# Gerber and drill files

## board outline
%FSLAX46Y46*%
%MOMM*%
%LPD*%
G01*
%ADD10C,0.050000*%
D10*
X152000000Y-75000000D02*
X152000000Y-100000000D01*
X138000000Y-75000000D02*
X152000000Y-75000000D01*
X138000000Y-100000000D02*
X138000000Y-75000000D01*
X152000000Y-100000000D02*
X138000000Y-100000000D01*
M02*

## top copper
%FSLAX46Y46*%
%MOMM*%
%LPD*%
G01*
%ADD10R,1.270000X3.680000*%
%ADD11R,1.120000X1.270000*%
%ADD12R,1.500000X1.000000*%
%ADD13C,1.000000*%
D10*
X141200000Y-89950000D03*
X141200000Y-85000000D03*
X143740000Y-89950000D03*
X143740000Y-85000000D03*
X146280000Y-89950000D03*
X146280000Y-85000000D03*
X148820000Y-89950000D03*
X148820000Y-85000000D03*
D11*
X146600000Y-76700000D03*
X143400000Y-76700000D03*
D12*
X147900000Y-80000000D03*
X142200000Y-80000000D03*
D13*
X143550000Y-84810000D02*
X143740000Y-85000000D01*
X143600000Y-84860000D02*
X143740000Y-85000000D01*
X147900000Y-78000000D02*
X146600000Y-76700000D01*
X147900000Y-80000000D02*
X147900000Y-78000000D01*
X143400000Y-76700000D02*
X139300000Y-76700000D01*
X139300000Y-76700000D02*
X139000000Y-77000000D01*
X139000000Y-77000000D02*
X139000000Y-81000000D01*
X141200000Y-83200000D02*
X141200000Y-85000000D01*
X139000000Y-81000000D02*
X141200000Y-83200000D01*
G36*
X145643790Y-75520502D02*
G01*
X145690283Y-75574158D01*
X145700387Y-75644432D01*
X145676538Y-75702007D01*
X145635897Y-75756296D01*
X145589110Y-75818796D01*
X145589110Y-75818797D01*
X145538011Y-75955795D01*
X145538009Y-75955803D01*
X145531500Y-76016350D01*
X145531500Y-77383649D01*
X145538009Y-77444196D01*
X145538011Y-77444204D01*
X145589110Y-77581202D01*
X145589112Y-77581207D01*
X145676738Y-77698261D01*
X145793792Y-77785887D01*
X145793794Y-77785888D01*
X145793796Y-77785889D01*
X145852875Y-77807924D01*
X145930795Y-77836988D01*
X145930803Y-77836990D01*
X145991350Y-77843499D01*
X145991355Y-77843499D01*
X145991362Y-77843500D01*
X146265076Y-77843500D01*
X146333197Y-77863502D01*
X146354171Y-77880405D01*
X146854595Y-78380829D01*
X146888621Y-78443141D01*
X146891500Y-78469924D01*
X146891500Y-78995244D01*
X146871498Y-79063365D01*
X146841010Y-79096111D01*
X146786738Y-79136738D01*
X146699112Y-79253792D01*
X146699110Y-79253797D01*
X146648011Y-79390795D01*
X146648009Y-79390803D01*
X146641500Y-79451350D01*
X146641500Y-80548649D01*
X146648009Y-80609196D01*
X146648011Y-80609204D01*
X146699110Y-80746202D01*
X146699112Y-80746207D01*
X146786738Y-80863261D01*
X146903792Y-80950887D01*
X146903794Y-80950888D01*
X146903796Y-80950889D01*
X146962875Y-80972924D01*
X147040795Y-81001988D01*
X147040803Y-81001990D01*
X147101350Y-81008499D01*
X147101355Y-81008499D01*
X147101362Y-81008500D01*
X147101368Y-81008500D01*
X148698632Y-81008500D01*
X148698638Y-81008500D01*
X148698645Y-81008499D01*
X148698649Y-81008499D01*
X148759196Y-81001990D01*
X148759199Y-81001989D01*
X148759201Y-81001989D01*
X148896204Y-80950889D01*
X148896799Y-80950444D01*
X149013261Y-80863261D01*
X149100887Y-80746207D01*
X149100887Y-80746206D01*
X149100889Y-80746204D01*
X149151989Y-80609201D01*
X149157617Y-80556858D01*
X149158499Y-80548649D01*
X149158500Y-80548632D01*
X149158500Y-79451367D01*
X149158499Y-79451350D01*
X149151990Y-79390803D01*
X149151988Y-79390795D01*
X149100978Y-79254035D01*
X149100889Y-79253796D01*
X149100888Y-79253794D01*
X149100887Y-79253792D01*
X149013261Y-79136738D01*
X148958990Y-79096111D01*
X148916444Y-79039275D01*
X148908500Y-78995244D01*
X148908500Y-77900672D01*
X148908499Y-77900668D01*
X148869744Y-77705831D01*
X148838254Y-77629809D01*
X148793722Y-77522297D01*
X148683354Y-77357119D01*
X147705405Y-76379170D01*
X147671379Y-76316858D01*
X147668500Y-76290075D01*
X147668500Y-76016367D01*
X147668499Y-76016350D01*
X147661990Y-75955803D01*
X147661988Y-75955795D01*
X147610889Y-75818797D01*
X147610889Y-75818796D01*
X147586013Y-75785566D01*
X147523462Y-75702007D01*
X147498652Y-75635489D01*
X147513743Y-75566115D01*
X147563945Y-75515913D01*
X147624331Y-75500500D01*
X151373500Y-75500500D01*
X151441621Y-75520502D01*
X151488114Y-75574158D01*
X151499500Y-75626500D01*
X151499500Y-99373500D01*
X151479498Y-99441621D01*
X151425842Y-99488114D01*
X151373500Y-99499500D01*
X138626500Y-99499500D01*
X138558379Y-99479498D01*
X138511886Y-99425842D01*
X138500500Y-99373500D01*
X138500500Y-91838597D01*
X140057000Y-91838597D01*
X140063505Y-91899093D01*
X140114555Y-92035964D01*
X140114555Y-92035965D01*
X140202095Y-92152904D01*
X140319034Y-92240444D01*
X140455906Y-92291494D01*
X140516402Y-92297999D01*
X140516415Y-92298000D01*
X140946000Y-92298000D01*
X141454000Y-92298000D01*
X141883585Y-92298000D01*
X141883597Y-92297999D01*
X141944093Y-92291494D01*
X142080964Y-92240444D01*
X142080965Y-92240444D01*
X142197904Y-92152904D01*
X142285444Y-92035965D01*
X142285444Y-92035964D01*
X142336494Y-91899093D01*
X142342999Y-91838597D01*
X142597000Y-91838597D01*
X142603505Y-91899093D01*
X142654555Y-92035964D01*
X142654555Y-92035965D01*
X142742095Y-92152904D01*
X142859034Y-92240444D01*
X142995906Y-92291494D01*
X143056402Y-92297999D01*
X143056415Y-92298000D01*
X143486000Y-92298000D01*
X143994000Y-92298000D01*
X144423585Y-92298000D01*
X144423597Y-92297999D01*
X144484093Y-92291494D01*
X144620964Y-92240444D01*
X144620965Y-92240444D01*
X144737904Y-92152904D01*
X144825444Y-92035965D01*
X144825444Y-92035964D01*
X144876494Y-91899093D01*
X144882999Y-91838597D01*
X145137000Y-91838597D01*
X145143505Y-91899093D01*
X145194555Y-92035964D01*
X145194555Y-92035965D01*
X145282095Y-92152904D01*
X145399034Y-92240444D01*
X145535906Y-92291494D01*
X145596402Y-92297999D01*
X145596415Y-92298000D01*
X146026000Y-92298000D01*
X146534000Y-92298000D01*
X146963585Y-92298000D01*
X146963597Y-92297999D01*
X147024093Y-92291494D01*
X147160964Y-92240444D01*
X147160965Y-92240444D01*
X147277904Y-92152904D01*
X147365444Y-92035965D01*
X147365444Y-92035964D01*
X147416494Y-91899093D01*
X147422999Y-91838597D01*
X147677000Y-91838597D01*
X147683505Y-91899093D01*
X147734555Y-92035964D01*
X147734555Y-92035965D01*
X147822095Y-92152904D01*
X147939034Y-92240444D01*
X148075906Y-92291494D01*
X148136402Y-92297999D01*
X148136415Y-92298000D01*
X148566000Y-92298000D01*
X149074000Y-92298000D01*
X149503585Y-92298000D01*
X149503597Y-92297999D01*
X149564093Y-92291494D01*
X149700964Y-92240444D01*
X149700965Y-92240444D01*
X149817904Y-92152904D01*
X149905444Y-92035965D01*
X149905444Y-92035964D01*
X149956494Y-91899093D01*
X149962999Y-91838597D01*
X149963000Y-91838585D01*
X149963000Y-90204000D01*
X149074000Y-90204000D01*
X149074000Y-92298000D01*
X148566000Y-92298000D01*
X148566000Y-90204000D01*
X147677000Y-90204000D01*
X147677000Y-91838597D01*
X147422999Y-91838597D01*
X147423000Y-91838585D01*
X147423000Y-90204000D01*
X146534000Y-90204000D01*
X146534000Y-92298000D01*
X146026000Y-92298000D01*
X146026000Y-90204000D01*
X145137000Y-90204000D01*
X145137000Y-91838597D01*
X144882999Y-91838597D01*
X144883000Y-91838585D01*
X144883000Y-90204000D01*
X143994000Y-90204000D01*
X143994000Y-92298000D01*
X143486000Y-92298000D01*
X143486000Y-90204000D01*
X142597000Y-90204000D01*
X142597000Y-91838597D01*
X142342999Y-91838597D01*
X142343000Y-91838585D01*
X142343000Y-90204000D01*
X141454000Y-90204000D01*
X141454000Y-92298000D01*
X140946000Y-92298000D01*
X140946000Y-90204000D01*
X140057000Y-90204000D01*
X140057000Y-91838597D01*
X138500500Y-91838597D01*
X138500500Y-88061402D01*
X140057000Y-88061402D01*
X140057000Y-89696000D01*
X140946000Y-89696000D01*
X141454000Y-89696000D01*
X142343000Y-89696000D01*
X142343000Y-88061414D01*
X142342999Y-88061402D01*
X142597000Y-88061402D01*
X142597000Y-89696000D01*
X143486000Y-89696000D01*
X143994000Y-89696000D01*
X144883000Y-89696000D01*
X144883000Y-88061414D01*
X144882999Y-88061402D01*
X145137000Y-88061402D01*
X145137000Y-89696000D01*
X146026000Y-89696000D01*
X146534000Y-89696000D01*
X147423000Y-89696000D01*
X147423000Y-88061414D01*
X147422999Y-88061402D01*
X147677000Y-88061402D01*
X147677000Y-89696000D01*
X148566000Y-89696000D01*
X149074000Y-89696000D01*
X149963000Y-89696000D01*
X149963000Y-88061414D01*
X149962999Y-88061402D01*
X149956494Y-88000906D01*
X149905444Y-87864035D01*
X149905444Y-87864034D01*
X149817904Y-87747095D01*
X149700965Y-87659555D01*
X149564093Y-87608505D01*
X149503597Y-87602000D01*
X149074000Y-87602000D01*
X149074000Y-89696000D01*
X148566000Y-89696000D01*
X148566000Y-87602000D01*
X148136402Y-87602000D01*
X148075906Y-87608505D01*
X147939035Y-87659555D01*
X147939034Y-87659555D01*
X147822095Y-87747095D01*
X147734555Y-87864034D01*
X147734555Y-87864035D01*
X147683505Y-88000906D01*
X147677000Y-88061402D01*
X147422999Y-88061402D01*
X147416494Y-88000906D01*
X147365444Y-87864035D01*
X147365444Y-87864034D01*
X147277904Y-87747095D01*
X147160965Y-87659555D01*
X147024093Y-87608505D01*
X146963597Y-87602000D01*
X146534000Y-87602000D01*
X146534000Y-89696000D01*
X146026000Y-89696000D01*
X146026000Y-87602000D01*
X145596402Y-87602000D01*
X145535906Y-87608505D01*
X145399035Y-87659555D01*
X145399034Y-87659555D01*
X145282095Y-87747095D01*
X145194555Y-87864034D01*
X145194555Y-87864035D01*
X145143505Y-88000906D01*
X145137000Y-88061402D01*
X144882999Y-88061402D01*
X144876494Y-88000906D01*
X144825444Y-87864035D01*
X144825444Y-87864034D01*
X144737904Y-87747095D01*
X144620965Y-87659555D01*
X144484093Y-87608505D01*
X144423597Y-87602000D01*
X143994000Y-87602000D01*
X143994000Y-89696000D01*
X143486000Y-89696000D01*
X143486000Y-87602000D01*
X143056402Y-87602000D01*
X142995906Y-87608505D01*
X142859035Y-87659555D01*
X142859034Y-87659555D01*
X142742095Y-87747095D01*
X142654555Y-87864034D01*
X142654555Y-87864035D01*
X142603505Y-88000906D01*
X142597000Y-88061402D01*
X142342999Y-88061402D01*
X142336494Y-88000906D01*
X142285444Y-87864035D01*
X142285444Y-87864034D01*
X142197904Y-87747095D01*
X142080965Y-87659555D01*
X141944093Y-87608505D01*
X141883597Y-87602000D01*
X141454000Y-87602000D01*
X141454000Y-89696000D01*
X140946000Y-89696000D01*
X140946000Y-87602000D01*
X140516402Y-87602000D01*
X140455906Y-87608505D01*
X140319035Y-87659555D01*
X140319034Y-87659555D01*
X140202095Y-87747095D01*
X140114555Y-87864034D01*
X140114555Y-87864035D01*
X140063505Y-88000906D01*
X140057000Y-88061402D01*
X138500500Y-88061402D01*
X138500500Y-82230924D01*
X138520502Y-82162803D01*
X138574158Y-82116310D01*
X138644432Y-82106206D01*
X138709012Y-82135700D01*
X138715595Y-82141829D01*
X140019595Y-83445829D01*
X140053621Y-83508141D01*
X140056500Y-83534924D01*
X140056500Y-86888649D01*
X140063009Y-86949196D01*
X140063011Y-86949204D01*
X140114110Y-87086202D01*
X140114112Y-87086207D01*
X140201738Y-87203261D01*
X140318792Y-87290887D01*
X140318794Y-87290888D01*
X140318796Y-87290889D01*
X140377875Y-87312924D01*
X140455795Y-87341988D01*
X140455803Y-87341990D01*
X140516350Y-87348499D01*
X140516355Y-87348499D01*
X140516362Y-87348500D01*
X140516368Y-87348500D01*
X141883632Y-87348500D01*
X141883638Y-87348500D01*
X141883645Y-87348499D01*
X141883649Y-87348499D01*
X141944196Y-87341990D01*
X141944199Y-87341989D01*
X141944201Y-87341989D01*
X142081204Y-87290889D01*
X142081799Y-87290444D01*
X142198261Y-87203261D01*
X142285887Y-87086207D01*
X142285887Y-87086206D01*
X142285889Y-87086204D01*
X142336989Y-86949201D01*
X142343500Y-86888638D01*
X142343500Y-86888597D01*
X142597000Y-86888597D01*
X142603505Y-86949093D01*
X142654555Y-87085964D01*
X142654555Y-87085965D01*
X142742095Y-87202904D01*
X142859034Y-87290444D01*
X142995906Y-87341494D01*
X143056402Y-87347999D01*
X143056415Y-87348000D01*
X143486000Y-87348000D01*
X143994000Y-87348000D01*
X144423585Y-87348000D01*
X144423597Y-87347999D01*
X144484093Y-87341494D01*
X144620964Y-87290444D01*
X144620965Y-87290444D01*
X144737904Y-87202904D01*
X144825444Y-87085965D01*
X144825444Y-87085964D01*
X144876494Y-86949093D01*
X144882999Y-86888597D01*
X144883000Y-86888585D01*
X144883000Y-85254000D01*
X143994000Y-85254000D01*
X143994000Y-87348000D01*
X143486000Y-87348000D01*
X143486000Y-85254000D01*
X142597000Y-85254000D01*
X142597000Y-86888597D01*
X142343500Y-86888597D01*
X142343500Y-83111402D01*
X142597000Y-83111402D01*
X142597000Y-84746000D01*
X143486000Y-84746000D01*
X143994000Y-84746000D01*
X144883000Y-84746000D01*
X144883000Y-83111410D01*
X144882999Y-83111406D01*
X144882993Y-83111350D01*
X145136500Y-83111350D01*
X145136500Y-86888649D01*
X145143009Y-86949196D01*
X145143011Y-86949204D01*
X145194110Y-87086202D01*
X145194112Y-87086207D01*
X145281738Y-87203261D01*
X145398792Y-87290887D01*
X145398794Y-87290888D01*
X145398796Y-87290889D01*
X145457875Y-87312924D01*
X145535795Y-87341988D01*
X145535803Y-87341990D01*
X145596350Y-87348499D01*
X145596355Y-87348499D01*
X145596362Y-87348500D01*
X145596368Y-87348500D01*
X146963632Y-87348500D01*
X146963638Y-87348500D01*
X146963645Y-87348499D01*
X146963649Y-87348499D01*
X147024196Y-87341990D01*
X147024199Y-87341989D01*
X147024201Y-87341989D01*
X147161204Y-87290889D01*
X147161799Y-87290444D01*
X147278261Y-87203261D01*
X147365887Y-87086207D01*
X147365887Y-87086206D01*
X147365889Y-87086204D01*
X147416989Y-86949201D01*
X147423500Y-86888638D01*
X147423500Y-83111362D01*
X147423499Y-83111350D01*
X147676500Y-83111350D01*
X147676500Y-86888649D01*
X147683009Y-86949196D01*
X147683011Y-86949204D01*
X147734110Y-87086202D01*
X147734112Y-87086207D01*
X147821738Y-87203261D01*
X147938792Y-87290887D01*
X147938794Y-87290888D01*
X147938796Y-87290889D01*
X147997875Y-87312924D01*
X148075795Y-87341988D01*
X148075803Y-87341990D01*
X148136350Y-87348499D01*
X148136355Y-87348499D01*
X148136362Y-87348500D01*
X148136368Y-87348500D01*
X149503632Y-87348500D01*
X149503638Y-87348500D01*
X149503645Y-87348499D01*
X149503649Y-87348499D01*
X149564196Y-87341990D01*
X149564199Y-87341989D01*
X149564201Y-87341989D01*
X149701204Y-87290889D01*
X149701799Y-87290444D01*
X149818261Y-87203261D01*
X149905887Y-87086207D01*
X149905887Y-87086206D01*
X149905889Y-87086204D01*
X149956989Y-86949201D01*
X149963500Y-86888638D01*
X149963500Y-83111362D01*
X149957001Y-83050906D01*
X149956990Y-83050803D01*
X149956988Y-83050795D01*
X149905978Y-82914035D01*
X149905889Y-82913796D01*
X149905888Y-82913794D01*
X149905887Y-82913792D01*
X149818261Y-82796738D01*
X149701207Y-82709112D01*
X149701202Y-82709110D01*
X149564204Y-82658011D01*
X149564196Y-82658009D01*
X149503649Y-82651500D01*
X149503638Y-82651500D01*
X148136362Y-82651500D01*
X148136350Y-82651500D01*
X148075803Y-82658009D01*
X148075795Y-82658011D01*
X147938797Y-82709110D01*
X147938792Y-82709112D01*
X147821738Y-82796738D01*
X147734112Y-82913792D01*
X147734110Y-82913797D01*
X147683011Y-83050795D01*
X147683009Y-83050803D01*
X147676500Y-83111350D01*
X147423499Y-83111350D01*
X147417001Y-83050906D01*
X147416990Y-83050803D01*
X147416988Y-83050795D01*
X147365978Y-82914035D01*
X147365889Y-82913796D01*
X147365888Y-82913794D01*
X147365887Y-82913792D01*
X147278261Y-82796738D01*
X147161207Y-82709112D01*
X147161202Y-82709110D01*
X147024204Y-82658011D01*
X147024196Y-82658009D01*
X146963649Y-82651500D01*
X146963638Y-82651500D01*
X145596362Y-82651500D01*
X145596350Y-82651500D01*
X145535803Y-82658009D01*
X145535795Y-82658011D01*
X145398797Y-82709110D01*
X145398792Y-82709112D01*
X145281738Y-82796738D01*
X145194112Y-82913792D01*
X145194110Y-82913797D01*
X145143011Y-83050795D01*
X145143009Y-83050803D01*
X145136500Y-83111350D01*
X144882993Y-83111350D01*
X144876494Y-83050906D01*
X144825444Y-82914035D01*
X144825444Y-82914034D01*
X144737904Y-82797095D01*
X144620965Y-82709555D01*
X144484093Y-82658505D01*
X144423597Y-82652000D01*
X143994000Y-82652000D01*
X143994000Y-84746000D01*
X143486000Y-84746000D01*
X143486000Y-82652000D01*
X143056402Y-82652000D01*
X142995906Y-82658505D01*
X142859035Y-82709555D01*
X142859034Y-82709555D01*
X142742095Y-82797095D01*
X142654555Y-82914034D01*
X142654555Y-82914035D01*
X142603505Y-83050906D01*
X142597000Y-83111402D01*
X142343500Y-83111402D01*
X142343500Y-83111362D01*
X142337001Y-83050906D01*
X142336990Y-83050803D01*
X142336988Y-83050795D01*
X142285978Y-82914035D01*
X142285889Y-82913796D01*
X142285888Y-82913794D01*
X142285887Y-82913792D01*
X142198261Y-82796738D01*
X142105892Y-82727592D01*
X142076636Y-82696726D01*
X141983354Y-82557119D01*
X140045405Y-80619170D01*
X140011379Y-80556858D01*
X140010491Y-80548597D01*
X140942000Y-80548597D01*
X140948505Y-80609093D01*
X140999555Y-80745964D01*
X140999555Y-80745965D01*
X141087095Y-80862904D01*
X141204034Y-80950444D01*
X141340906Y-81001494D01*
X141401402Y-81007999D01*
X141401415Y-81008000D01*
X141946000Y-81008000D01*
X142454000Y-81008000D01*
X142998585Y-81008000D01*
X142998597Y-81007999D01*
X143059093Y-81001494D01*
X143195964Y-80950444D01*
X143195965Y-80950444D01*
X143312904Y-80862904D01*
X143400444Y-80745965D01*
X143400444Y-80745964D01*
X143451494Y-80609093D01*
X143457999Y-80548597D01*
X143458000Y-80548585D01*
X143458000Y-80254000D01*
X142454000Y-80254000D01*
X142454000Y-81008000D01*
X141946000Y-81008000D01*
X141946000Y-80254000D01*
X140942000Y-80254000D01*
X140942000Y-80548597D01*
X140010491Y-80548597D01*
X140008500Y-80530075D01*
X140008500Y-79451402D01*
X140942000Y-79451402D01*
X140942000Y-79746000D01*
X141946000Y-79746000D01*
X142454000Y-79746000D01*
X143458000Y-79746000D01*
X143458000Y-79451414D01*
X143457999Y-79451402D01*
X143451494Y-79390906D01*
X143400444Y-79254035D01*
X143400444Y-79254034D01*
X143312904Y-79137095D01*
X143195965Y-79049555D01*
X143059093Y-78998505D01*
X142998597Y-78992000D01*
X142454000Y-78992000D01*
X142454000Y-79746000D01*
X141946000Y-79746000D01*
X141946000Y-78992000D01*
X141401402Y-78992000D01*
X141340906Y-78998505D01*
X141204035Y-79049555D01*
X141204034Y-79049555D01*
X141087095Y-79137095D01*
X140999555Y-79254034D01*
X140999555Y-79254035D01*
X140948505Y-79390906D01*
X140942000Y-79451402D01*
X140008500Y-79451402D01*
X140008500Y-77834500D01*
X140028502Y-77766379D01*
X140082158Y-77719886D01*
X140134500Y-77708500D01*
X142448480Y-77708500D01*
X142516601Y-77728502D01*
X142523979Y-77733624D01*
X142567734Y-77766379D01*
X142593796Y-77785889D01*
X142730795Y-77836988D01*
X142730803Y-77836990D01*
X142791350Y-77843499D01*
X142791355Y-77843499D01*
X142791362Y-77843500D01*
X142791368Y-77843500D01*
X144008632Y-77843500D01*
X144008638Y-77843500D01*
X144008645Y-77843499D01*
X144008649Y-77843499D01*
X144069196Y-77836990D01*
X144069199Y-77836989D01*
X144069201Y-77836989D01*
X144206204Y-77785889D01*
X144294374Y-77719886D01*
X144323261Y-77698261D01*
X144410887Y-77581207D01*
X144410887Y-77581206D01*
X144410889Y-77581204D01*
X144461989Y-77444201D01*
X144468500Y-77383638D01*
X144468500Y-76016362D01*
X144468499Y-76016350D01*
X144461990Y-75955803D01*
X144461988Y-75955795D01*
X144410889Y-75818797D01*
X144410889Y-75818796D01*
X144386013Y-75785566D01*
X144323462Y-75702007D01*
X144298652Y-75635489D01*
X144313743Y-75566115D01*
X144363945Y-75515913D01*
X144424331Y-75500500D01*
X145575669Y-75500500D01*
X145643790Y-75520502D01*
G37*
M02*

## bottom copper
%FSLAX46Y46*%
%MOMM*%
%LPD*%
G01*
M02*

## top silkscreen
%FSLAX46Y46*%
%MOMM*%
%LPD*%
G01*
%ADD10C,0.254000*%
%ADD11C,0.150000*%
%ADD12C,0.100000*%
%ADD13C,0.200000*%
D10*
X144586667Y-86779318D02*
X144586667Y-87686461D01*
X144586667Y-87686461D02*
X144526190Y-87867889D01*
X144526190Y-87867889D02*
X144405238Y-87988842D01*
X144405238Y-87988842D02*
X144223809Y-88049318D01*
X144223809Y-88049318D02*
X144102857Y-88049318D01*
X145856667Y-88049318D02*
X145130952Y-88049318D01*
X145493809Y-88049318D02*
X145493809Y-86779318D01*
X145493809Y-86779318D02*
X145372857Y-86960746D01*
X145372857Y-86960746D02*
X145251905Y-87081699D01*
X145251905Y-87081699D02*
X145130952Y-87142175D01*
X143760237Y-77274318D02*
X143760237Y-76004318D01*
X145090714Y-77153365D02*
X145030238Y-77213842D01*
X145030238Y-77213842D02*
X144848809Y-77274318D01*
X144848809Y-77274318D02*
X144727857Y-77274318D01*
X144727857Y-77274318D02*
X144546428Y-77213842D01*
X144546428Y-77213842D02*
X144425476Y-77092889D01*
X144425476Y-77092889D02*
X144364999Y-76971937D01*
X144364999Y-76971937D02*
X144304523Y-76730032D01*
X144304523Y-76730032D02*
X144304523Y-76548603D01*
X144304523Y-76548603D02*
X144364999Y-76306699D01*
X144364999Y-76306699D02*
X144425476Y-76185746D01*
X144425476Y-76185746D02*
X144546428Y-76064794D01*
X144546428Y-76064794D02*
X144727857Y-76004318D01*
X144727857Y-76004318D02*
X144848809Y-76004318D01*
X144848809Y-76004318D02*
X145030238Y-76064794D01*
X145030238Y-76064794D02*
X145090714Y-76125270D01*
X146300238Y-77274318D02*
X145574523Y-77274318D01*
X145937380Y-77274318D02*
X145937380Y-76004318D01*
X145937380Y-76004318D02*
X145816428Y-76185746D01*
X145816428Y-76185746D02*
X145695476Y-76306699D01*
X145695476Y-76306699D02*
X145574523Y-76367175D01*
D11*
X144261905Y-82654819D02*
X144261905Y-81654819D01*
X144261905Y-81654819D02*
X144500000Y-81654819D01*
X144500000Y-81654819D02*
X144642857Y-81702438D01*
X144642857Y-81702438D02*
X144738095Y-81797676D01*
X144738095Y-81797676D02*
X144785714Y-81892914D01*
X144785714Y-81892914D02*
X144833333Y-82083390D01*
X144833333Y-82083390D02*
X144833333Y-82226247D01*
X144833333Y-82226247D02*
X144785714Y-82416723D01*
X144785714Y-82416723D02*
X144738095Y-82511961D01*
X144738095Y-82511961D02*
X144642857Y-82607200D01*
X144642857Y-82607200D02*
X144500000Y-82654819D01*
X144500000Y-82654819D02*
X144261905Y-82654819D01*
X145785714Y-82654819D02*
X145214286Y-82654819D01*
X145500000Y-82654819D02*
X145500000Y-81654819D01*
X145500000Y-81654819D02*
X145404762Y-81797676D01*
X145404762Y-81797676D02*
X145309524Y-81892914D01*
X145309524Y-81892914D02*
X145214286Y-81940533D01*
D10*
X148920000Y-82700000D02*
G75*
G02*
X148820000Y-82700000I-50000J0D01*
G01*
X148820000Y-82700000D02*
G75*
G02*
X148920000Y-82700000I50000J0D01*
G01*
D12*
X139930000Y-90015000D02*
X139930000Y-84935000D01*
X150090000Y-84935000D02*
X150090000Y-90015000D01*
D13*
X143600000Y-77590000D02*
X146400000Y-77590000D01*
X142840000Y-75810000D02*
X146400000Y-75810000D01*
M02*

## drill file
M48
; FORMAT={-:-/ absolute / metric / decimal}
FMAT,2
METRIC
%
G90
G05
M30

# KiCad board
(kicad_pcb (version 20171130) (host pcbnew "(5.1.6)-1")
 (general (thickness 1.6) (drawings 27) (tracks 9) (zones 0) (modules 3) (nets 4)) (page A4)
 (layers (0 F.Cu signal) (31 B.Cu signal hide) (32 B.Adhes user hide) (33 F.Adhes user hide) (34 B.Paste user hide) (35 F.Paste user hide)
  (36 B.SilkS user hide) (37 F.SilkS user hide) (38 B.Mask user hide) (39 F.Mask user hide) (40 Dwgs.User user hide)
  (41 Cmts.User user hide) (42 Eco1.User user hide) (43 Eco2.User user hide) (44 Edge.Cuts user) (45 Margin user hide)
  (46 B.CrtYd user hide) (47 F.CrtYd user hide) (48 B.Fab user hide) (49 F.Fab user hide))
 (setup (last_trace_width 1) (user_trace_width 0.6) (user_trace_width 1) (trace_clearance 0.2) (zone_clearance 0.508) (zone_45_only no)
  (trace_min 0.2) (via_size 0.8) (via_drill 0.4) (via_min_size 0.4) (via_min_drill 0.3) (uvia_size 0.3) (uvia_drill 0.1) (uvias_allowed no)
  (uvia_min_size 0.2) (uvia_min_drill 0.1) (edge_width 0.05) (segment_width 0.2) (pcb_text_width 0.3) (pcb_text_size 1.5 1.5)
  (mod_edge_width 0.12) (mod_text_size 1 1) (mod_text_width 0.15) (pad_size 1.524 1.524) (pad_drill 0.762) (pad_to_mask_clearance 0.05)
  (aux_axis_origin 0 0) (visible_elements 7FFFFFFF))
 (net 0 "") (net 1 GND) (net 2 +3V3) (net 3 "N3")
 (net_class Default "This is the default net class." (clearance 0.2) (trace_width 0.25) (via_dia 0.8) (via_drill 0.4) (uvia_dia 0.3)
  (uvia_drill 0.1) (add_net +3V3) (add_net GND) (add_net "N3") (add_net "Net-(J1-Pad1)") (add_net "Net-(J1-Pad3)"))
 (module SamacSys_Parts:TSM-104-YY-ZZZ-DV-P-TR (layer F.Cu) (at 145.01 87.475)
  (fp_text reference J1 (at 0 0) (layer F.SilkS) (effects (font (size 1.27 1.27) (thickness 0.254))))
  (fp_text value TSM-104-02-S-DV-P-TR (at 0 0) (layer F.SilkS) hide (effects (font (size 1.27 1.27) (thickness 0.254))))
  (fp_circle (center 3.86 -4.775) (end 3.81 -4.775) (layer F.SilkS) (width 0.254))
  (fp_line (start -5.08 2.54) (end -5.08 -2.54) (layer F.SilkS) (width 0.1))
  (fp_line (start 5.08 -2.54) (end 5.08 2.54) (layer F.SilkS) (width 0.1))
  (pad 8 smd rect (at -3.81 2.475) (size 1.27 3.68) (layers F.Cu F.Paste F.Mask) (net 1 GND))
  (pad 7 smd rect (at -3.81 -2.475) (size 1.27 3.68) (layers F.Cu F.Paste F.Mask) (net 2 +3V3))
  (pad 6 smd rect (at -1.27 2.475) (size 1.27 3.68) (layers F.Cu F.Paste F.Mask) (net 1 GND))
  (pad 5 smd rect (at -1.27 -2.475) (size 1.27 3.68) (layers F.Cu F.Paste F.Mask) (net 1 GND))
  (pad 4 smd rect (at 1.27 2.475) (size 1.27 3.68) (layers F.Cu F.Paste F.Mask) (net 1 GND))
  (pad 3 smd rect (at 1.27 -2.475) (size 1.27 3.68) (layers F.Cu F.Paste F.Mask))
  (pad 2 smd rect (at 3.81 2.475) (size 1.27 3.68) (layers F.Cu F.Paste F.Mask) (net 1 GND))
  (pad 1 smd rect (at 3.81 -2.475) (size 1.27 3.68) (layers F.Cu F.Paste F.Mask)))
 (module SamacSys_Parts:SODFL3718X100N (layer F.Cu) (at 145 76.7)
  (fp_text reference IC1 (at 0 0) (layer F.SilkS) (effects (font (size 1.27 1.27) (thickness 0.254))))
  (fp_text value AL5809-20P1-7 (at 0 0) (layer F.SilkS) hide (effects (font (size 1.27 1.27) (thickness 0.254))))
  (fp_line (start -1.4 0.89) (end 1.4 0.89) (layer F.SilkS) (width 0.2))
  (fp_line (start -2.16 -0.89) (end 1.4 -0.89) (layer F.SilkS) (width 0.2))
  (pad 2 smd rect (at 1.6 0) (size 1.12 1.27) (layers F.Cu F.Paste F.Mask) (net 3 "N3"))
  (pad 1 smd rect (at -1.6 0) (size 1.12 1.27) (layers F.Cu F.Paste F.Mask) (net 2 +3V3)))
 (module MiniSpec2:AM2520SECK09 (layer F.Cu) (at 145 80)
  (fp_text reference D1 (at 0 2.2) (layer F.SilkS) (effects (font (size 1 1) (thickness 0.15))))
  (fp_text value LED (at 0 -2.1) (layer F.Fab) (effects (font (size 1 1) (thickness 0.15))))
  (pad 2 smd rect (at 2.9 0) (size 1.5 1) (layers F.Cu F.Paste F.Mask) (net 3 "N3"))
  (pad 1 smd rect (at -2.8 0) (size 1.5 1) (layers F.Cu F.Paste F.Mask) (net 1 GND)))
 (gr_line (start 152 75) (end 152 100) (layer Edge.Cuts) (width 0.05))
 (gr_line (start 138 75) (end 152 75) (layer Edge.Cuts) (width 0.05))
 (gr_line (start 138 100) (end 138 75) (layer Edge.Cuts) (width 0.05))
 (gr_line (start 152 100) (end 138 100) (layer Edge.Cuts) (width 0.05))
 (segment (start 143.55 84.81) (end 143.74 85) (width 1) (layer F.Cu) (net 1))
 (segment (start 143.6 84.86) (end 143.74 85) (width 1) (layer F.Cu) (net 1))
 (segment (start 147.9 78) (end 146.6 76.7) (width 1) (layer F.Cu) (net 3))
 (segment (start 147.9 80) (end 147.9 78) (width 1) (layer F.Cu) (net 3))
 (segment (start 143.4 76.7) (end 139.3 76.7) (width 1) (layer F.Cu) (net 2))
 (segment (start 139.3 76.7) (end 139 77) (width 1) (layer F.Cu) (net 2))
 (segment (start 139 77) (end 139 81) (width 1) (layer F.Cu) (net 2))
 (segment (start 141.2 83.2) (end 141.2 85) (width 1) (layer F.Cu) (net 2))
 (segment (start 139 81) (end 141.2 83.2) (width 1) (layer F.Cu) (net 2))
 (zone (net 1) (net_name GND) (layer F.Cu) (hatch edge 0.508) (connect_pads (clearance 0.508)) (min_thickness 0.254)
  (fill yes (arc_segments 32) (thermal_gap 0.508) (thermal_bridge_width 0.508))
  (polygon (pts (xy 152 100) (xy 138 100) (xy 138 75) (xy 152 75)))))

